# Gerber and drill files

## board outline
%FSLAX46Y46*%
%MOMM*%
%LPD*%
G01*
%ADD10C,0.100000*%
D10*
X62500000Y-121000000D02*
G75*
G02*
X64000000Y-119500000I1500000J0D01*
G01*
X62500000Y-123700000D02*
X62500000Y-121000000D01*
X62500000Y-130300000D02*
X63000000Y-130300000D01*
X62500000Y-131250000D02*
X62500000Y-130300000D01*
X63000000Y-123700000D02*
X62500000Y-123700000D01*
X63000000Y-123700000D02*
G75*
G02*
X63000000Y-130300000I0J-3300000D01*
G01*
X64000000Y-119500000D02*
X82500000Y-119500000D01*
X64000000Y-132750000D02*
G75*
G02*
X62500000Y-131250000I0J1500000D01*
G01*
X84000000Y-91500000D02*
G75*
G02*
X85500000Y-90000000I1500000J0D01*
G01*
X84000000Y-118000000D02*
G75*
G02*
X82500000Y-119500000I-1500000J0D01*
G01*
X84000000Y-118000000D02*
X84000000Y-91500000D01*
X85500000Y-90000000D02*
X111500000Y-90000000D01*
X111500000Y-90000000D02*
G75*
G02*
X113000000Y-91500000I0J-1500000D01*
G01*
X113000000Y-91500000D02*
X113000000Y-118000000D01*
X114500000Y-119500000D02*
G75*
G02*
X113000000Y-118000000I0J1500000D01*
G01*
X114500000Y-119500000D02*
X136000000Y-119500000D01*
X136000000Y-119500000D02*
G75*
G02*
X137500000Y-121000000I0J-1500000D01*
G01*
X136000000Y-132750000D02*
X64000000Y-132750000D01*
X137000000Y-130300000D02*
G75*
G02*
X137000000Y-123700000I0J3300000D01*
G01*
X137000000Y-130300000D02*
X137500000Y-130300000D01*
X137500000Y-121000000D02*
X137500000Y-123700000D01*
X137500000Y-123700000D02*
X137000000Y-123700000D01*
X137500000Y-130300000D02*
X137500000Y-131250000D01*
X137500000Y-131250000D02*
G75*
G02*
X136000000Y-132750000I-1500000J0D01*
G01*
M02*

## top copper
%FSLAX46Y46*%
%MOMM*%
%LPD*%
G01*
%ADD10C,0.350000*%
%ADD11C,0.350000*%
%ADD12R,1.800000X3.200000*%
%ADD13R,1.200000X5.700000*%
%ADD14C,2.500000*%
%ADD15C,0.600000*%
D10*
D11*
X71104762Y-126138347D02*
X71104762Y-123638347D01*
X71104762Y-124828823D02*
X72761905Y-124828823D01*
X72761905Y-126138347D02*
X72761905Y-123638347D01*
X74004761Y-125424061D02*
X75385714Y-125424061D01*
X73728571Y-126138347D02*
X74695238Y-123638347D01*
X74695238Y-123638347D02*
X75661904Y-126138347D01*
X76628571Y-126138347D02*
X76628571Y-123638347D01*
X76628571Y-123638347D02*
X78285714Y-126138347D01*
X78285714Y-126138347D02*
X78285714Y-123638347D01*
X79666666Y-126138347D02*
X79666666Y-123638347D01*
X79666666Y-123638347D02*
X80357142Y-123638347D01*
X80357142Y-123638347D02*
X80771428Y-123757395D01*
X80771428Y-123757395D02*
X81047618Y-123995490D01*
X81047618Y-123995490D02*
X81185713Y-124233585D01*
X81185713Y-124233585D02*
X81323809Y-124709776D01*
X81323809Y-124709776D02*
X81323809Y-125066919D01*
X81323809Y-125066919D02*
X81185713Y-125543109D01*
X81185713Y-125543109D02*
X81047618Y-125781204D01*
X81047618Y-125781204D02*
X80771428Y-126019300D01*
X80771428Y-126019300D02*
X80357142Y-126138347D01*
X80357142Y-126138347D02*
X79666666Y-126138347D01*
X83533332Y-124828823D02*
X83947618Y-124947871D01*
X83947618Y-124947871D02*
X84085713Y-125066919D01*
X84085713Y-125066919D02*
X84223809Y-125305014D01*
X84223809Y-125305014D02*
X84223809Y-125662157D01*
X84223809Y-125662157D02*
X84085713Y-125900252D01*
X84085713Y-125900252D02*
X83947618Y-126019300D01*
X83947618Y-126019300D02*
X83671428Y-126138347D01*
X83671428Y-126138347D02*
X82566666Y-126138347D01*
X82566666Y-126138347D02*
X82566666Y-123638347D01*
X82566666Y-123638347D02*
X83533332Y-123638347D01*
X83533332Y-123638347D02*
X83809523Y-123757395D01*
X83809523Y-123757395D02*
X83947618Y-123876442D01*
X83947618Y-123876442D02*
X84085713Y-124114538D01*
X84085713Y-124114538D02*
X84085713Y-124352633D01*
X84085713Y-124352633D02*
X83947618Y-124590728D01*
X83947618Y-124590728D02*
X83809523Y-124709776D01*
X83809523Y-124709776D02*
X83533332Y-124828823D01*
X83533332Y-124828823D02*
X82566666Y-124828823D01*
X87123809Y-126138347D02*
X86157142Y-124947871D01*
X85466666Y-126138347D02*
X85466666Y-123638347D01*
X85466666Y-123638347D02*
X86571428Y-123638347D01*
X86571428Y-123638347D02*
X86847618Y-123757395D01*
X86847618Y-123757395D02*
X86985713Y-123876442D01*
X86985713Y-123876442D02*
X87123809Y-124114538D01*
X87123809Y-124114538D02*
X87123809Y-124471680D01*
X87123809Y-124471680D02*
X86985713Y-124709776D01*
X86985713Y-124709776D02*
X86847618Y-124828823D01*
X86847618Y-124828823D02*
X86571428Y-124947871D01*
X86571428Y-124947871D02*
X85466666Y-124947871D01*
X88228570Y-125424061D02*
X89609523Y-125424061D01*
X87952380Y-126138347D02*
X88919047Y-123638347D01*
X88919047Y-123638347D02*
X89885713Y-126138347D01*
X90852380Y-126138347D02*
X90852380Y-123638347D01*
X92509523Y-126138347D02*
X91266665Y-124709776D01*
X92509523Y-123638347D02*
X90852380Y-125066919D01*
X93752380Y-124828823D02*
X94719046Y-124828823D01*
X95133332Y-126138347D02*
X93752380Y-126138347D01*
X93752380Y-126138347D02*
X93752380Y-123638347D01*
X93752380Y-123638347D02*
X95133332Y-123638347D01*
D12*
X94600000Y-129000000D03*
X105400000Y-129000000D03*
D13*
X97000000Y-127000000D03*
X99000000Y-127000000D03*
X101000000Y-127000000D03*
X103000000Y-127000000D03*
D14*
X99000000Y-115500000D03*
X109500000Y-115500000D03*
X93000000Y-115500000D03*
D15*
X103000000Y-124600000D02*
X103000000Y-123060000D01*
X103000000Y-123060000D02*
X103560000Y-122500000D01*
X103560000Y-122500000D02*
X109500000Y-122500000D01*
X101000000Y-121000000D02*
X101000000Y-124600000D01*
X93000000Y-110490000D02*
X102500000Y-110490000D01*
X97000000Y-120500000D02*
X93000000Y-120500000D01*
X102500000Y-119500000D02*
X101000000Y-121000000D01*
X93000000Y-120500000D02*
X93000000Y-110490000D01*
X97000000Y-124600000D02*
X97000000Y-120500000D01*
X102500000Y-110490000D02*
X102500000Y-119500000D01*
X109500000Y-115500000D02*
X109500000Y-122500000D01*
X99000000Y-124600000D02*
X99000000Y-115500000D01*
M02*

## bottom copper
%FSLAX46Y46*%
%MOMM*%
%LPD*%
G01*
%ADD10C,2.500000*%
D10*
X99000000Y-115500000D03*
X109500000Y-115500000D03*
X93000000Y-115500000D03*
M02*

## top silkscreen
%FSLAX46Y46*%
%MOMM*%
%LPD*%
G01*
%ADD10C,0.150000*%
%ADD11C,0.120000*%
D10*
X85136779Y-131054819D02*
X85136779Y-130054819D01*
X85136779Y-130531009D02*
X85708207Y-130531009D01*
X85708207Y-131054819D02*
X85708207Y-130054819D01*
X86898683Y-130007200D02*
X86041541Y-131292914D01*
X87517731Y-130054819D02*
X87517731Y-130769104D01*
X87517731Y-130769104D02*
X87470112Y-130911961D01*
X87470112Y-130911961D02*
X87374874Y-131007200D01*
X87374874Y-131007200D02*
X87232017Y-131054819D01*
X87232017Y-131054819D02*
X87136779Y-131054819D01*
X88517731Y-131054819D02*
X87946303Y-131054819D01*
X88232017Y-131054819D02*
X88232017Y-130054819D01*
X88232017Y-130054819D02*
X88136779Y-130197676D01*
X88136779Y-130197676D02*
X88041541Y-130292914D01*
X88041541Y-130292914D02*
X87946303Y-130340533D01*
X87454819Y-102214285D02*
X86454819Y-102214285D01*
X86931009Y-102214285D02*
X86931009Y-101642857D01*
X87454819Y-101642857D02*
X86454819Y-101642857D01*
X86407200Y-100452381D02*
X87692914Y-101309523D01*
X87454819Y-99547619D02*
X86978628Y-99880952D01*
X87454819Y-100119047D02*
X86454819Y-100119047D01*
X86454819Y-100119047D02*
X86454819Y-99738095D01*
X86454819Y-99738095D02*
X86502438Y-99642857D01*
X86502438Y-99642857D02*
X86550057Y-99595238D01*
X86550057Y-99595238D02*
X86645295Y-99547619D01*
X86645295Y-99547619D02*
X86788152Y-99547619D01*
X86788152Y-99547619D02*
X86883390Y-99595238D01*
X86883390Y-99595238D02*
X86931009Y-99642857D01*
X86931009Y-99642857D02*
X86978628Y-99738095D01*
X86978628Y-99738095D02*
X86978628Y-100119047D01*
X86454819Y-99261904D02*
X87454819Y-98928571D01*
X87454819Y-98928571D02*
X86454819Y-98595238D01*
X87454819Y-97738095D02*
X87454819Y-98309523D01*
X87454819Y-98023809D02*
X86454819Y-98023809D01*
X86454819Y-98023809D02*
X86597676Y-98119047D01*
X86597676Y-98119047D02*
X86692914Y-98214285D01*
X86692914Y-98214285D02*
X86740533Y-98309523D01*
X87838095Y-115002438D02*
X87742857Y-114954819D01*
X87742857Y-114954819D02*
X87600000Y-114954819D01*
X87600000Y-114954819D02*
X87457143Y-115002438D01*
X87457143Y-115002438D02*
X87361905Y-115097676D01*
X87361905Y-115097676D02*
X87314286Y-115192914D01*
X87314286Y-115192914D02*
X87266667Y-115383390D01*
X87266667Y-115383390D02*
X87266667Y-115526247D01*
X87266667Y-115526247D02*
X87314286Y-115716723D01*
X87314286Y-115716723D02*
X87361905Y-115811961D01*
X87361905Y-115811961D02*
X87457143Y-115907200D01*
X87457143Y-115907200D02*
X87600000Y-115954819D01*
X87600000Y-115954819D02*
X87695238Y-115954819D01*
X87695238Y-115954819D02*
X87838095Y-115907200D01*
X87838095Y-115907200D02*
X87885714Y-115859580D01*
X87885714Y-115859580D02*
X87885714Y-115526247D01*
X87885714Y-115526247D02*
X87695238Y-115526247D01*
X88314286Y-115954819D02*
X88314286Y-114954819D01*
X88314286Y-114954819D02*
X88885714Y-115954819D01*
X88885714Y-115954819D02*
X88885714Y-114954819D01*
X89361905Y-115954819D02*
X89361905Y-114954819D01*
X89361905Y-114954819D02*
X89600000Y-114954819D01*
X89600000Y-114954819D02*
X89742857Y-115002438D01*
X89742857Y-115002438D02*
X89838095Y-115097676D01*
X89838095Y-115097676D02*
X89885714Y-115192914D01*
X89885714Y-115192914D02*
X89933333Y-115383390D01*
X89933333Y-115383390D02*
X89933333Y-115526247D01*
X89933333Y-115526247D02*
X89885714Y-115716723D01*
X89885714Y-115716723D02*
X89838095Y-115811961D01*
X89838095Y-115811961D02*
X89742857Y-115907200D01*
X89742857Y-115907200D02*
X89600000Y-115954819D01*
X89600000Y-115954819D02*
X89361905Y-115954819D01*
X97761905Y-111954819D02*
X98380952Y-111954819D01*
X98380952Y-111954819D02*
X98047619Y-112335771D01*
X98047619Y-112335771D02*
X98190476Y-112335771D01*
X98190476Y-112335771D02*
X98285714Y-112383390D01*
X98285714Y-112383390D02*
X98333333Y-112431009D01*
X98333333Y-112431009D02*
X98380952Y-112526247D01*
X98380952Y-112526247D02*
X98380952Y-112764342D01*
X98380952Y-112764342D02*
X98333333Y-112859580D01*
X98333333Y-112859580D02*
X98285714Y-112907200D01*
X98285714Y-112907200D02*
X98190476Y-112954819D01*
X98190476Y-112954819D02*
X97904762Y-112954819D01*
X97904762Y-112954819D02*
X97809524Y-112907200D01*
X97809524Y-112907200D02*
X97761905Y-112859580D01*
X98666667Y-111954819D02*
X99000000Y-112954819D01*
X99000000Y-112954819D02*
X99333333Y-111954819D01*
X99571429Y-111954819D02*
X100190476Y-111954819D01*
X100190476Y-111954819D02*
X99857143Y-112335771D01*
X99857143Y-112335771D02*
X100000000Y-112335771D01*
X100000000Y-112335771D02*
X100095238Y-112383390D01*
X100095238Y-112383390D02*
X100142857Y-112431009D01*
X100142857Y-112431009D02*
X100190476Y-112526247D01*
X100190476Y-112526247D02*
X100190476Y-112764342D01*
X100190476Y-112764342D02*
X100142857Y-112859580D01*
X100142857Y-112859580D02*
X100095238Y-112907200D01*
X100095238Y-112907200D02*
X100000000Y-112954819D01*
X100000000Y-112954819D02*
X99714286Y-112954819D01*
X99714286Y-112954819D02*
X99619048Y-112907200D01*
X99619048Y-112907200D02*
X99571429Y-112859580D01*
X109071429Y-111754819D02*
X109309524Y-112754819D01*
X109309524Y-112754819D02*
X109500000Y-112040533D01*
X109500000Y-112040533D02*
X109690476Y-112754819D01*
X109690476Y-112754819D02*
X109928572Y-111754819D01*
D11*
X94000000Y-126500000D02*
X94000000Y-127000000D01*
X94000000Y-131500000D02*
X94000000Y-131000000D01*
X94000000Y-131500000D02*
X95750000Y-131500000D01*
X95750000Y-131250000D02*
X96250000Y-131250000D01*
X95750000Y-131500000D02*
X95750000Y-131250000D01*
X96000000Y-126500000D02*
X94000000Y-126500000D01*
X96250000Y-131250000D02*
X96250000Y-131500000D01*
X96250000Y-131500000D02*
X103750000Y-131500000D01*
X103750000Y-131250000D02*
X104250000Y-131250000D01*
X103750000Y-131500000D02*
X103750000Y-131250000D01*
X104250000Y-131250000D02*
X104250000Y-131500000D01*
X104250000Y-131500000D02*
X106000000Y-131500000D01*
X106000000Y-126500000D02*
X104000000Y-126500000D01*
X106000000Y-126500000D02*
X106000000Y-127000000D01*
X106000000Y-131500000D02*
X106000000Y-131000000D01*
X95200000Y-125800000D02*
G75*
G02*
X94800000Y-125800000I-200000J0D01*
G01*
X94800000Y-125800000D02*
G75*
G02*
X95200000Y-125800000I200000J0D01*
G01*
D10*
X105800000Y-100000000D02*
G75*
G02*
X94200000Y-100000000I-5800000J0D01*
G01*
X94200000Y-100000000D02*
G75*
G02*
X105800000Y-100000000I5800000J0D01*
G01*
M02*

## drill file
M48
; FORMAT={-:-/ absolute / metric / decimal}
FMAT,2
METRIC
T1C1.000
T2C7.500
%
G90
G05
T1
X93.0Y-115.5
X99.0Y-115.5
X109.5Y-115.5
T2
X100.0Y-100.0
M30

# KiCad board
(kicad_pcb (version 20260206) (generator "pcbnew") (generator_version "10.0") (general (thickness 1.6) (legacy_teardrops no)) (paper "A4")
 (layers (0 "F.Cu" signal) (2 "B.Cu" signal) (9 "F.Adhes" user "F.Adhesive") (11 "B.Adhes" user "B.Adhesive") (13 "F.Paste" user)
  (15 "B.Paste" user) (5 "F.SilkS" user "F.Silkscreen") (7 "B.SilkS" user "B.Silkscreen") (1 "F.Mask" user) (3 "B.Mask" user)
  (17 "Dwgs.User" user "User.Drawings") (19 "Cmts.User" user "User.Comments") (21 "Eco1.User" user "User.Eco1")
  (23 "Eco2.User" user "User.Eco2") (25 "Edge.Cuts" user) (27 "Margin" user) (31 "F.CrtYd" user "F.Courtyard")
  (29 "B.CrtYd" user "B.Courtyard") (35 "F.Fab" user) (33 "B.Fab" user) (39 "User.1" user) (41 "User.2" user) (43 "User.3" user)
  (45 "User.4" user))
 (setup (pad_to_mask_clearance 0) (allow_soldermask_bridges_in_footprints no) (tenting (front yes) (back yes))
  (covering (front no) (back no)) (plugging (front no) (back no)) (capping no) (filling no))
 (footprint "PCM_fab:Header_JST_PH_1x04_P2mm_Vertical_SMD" (layer "F.Cu") (at 98 127 90)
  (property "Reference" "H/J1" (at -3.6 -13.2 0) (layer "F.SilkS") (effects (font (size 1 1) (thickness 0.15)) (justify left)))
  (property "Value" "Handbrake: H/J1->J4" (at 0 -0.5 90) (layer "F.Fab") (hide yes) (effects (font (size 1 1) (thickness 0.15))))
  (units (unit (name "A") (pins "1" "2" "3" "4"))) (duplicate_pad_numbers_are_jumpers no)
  (fp_line (start 0.5 -4) (end 0 -4) (stroke (width 0.12) (type solid)) (layer "F.SilkS"))
  (fp_line (start -4.5 -4) (end -4 -4) (stroke (width 0.12) (type solid)) (layer "F.SilkS"))
  (fp_line (start -4.5 -4) (end -4.5 -2.25) (stroke (width 0.12) (type solid)) (layer "F.SilkS"))
  (fp_line (start -4.25 -2.25) (end -4.25 -1.75) (stroke (width 0.12) (type solid)) (layer "F.SilkS"))
  (fp_line (start -4.5 -2.25) (end -4.25 -2.25) (stroke (width 0.12) (type solid)) (layer "F.SilkS"))
  (fp_line (start 0.5 -2) (end 0.5 -4) (stroke (width 0.12) (type solid)) (layer "F.SilkS"))
  (fp_line (start -4.25 -1.75) (end -4.5 -1.75) (stroke (width 0.12) (type solid)) (layer "F.SilkS"))
  (fp_line (start -4.5 -1.75) (end -4.5 5.75) (stroke (width 0.12) (type solid)) (layer "F.SilkS"))
  (fp_line (start -4.25 5.75) (end -4.25 6.25) (stroke (width 0.12) (type solid)) (layer "F.SilkS"))
  (fp_line (start -4.5 5.75) (end -4.25 5.75) (stroke (width 0.12) (type solid)) (layer "F.SilkS"))
  (fp_line (start -4.25 6.25) (end -4.5 6.25) (stroke (width 0.12) (type solid)) (layer "F.SilkS"))
  (fp_line (start -4.5 6.25) (end -4.5 8) (stroke (width 0.12) (type solid)) (layer "F.SilkS"))
  (fp_line (start 0.5 8) (end 0.5 6) (stroke (width 0.12) (type solid)) (layer "F.SilkS"))
  (fp_line (start 0.5 8) (end 0 8) (stroke (width 0.12) (type solid)) (layer "F.SilkS"))
  (fp_line (start -4.5 8) (end -4 8) (stroke (width 0.12) (type solid)) (layer "F.SilkS"))
  (fp_circle (center 1.2 -3) (end 1.4 -3) (stroke (width 0.12) (type solid)) (fill no) (layer "F.SilkS"))
  (pad "" smd rect (at -2 -3.4 90) (size 3.2 1.8) (layers "F.Cu" "F.Mask" "F.Paste"))
  (pad "" smd rect (at -2 7.4 90) (size 3.2 1.8) (layers "F.Cu" "F.Mask" "F.Paste"))
  (pad "1" smd rect (at 0 -1 90) (size 5.7 1.2) (layers "F.Cu" "F.Mask" "F.Paste") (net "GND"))
  (pad "2" smd rect (at 0 1 90) (size 5.7 1.2) (layers "F.Cu" "F.Mask" "F.Paste") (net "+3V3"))
  (pad "3" smd rect (at 0 3 90) (size 5.7 1.2) (layers "F.Cu" "F.Mask" "F.Paste") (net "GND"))
  (pad "4" smd rect (at 0 5 90) (size 5.7 1.2) (layers "F.Cu" "F.Mask" "F.Paste") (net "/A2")))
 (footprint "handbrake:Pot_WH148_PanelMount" (layer "F.Cu") (at 100 100)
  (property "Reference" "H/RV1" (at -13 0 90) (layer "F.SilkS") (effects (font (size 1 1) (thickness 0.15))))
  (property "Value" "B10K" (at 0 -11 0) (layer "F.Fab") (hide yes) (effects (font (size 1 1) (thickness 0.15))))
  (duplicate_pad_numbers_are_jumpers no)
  (fp_circle (center 0 0) (end 5.8 0) (stroke (width 0.15) (type solid)) (fill no) (layer "F.SilkS"))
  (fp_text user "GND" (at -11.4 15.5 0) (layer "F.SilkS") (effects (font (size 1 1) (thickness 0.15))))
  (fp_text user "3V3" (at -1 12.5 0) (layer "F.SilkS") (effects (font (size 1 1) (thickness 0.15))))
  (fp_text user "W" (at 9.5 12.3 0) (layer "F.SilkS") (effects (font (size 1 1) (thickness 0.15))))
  (pad "" np_thru_hole circle (at 0 0) (size 7.5 7.5) (drill 7.5) (layers "*.Cu" "*.Mask"))
  (pad "1" thru_hole circle (at -1 15.5) (size 2.5 2.5) (drill 1) (layers "*.Cu" "*.Mask") (remove_unused_layers no) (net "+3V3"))
  (pad "2" thru_hole circle (at 9.5 15.5) (size 2.5 2.5) (drill 1) (layers "*.Cu" "*.Mask") (remove_unused_layers no) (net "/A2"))
  (pad "3" thru_hole circle (at -7 15.5) (size 2.5 2.5) (drill 1) (layers "*.Cu" "*.Mask") (remove_unused_layers no) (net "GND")))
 (gr_arc (start 62.5 121) (mid 62.939339 119.939339) (end 64 119.5) (stroke (width 0.1) (type default)) (layer "Edge.Cuts"))
 (gr_line (start 62.5 123.7) (end 62.5 121) (stroke (width 0.1) (type default)) (layer "Edge.Cuts"))
 (gr_line (start 62.5 130.3) (end 63 130.3) (stroke (width 0.1) (type default)) (layer "Edge.Cuts"))
 (gr_line (start 62.5 131.25) (end 62.5 130.3) (stroke (width 0.1) (type default)) (layer "Edge.Cuts"))
 (gr_line (start 63 123.7) (end 62.5 123.7) (stroke (width 0.1) (type default)) (layer "Edge.Cuts"))
 (gr_arc (start 63 123.7) (mid 66.3 127) (end 63 130.3) (stroke (width 0.1) (type default)) (layer "Edge.Cuts"))
 (gr_line (start 64 119.5) (end 82.5 119.5) (stroke (width 0.1) (type default)) (layer "Edge.Cuts"))
 (gr_arc (start 64 132.75) (mid 62.939339 132.31066) (end 62.5 131.25) (stroke (width 0.1) (type default)) (layer "Edge.Cuts"))
 (gr_arc (start 84 91.5) (mid 84.43934 90.43934) (end 85.5 90) (stroke (width 0.1) (type default)) (layer "Edge.Cuts"))
 (gr_arc (start 84 118) (mid 83.56066 119.06066) (end 82.5 119.5) (stroke (width 0.1) (type default)) (layer "Edge.Cuts"))
 (gr_line (start 84 118) (end 84 91.5) (stroke (width 0.1) (type default)) (layer "Edge.Cuts"))
 (gr_line (start 85.5 90) (end 111.5 90) (stroke (width 0.1) (type default)) (layer "Edge.Cuts"))
 (gr_arc (start 111.5 90) (mid 112.56066 90.43934) (end 113 91.5) (stroke (width 0.1) (type default)) (layer "Edge.Cuts"))
 (gr_line (start 113 91.5) (end 113 118) (stroke (width 0.1) (type default)) (layer "Edge.Cuts"))
 (gr_arc (start 114.5 119.5) (mid 113.43934 119.06066) (end 113 118) (stroke (width 0.1) (type default)) (layer "Edge.Cuts"))
 (gr_line (start 114.5 119.5) (end 136 119.5) (stroke (width 0.1) (type default)) (layer "Edge.Cuts"))
 (gr_arc (start 136 119.5) (mid 137.06066 119.939339) (end 137.5 121) (stroke (width 0.1) (type default)) (layer "Edge.Cuts"))
 (gr_line (start 136 132.75) (end 64 132.75) (stroke (width 0.1) (type default)) (layer "Edge.Cuts"))
 (gr_arc (start 137 130.3) (mid 133.7 127) (end 137 123.7) (stroke (width 0.1) (type default)) (layer "Edge.Cuts"))
 (gr_line (start 137 130.3) (end 137.5 130.3) (stroke (width 0.1) (type default)) (layer "Edge.Cuts"))
 (gr_line (start 137.5 121) (end 137.5 123.7) (stroke (width 0.1) (type default)) (layer "Edge.Cuts"))
 (gr_line (start 137.5 123.7) (end 137 123.7) (stroke (width 0.1) (type default)) (layer "Edge.Cuts"))
 (gr_line (start 137.5 130.3) (end 137.5 131.25) (stroke (width 0.1) (type default)) (layer "Edge.Cuts"))
 (gr_arc (start 137.5 131.25) (mid 137.06066 132.31066) (end 136 132.75) (stroke (width 0.1) (type default)) (layer "Edge.Cuts"))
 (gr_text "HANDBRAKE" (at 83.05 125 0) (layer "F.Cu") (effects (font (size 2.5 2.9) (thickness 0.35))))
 (segment (start 103 124.6) (end 103 123.06) (width 0.6) (layer "F.Cu") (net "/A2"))
 (segment (start 103 123.06) (end 103.56 122.5) (width 0.6) (layer "F.Cu") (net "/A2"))
 (segment (start 103.56 122.5) (end 109.5 122.5) (width 0.6) (layer "F.Cu") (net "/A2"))
 (segment (start 101 121) (end 101 124.6) (width 0.6) (layer "F.Cu") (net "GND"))
 (segment (start 93 110.49) (end 102.5 110.49) (width 0.6) (layer "F.Cu") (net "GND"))
 (segment (start 97 120.5) (end 93 120.5) (width 0.6) (layer "F.Cu") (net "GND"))
 (segment (start 102.5 119.5) (end 101 121) (width 0.6) (layer "F.Cu") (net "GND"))
 (segment (start 93 120.5) (end 93 110.49) (width 0.6) (layer "F.Cu") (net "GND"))
 (segment (start 97 124.6) (end 97 120.5) (width 0.6) (layer "F.Cu") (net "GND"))
 (segment (start 102.5 110.49) (end 102.5 119.5) (width 0.6) (layer "F.Cu") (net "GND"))
 (segment (start 109.5 115.5) (end 109.5 122.5) (width 0.6) (layer "F.Cu") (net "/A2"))
 (segment (start 99 124.6) (end 99 115.5) (width 0.6) (layer "F.Cu") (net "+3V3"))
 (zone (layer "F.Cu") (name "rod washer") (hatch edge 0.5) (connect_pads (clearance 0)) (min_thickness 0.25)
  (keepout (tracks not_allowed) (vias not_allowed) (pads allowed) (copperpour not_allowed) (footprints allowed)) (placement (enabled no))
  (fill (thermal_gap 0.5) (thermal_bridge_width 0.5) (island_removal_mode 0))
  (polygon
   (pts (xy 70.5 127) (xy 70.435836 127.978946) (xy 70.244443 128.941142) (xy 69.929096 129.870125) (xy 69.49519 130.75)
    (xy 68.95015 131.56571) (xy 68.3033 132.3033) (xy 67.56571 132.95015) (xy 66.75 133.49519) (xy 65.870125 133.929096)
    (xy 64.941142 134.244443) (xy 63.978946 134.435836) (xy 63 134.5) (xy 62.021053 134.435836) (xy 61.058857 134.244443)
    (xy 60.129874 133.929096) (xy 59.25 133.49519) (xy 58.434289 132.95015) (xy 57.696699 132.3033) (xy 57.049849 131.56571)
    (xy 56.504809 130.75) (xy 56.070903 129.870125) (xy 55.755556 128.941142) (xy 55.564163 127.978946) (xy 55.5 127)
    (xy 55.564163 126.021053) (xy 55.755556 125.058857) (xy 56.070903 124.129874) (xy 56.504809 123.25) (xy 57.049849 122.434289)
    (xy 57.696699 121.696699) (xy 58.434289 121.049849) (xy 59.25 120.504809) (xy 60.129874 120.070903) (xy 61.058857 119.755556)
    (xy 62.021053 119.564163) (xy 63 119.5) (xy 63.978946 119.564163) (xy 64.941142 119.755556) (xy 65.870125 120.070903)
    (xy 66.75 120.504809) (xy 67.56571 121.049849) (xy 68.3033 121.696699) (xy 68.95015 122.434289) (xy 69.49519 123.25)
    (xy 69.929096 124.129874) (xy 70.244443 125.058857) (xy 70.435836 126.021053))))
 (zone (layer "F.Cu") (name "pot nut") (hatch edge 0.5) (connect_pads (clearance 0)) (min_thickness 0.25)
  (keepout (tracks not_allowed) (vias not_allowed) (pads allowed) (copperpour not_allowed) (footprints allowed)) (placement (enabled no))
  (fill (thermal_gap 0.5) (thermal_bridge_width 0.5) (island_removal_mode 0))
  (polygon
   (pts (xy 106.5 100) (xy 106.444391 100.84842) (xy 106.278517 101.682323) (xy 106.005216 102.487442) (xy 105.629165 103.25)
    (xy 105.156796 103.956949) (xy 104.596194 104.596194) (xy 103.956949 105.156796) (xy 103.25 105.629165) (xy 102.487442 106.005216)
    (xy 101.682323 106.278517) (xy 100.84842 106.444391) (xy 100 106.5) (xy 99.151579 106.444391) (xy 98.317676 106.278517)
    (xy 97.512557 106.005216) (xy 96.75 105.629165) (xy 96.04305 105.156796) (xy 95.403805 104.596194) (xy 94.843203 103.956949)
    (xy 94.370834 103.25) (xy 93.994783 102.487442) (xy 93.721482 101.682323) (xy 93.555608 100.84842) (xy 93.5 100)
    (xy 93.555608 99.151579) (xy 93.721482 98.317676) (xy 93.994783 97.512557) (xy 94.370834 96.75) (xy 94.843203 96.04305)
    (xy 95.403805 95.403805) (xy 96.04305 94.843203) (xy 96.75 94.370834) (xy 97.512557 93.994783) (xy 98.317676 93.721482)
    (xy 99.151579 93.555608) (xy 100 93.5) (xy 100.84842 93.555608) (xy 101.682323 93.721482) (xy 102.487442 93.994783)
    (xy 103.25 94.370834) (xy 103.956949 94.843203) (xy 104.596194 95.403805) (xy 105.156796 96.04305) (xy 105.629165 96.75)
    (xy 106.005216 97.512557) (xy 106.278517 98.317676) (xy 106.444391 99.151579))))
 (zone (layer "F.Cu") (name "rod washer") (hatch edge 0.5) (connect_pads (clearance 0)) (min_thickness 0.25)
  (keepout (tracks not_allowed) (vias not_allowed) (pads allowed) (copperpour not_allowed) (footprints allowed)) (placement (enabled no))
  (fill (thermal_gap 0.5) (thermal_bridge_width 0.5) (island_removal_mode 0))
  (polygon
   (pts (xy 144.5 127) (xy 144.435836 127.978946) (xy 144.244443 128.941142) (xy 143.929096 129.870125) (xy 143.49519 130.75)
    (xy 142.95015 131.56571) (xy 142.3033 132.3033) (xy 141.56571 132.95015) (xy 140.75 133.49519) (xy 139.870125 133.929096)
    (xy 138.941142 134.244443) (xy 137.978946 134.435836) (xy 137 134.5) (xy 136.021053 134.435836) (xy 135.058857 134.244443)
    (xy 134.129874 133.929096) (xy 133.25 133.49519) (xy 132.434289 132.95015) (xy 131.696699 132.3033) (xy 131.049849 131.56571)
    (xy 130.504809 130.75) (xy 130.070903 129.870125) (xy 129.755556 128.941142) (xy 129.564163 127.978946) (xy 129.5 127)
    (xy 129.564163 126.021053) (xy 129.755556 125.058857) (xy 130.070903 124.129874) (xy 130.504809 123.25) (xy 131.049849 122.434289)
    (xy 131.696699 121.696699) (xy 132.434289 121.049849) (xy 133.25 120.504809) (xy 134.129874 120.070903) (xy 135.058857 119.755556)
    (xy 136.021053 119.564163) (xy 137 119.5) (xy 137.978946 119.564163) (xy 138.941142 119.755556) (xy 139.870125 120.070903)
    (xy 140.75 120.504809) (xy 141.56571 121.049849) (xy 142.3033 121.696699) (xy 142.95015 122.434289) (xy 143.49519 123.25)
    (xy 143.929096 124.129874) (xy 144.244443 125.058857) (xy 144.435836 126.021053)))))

